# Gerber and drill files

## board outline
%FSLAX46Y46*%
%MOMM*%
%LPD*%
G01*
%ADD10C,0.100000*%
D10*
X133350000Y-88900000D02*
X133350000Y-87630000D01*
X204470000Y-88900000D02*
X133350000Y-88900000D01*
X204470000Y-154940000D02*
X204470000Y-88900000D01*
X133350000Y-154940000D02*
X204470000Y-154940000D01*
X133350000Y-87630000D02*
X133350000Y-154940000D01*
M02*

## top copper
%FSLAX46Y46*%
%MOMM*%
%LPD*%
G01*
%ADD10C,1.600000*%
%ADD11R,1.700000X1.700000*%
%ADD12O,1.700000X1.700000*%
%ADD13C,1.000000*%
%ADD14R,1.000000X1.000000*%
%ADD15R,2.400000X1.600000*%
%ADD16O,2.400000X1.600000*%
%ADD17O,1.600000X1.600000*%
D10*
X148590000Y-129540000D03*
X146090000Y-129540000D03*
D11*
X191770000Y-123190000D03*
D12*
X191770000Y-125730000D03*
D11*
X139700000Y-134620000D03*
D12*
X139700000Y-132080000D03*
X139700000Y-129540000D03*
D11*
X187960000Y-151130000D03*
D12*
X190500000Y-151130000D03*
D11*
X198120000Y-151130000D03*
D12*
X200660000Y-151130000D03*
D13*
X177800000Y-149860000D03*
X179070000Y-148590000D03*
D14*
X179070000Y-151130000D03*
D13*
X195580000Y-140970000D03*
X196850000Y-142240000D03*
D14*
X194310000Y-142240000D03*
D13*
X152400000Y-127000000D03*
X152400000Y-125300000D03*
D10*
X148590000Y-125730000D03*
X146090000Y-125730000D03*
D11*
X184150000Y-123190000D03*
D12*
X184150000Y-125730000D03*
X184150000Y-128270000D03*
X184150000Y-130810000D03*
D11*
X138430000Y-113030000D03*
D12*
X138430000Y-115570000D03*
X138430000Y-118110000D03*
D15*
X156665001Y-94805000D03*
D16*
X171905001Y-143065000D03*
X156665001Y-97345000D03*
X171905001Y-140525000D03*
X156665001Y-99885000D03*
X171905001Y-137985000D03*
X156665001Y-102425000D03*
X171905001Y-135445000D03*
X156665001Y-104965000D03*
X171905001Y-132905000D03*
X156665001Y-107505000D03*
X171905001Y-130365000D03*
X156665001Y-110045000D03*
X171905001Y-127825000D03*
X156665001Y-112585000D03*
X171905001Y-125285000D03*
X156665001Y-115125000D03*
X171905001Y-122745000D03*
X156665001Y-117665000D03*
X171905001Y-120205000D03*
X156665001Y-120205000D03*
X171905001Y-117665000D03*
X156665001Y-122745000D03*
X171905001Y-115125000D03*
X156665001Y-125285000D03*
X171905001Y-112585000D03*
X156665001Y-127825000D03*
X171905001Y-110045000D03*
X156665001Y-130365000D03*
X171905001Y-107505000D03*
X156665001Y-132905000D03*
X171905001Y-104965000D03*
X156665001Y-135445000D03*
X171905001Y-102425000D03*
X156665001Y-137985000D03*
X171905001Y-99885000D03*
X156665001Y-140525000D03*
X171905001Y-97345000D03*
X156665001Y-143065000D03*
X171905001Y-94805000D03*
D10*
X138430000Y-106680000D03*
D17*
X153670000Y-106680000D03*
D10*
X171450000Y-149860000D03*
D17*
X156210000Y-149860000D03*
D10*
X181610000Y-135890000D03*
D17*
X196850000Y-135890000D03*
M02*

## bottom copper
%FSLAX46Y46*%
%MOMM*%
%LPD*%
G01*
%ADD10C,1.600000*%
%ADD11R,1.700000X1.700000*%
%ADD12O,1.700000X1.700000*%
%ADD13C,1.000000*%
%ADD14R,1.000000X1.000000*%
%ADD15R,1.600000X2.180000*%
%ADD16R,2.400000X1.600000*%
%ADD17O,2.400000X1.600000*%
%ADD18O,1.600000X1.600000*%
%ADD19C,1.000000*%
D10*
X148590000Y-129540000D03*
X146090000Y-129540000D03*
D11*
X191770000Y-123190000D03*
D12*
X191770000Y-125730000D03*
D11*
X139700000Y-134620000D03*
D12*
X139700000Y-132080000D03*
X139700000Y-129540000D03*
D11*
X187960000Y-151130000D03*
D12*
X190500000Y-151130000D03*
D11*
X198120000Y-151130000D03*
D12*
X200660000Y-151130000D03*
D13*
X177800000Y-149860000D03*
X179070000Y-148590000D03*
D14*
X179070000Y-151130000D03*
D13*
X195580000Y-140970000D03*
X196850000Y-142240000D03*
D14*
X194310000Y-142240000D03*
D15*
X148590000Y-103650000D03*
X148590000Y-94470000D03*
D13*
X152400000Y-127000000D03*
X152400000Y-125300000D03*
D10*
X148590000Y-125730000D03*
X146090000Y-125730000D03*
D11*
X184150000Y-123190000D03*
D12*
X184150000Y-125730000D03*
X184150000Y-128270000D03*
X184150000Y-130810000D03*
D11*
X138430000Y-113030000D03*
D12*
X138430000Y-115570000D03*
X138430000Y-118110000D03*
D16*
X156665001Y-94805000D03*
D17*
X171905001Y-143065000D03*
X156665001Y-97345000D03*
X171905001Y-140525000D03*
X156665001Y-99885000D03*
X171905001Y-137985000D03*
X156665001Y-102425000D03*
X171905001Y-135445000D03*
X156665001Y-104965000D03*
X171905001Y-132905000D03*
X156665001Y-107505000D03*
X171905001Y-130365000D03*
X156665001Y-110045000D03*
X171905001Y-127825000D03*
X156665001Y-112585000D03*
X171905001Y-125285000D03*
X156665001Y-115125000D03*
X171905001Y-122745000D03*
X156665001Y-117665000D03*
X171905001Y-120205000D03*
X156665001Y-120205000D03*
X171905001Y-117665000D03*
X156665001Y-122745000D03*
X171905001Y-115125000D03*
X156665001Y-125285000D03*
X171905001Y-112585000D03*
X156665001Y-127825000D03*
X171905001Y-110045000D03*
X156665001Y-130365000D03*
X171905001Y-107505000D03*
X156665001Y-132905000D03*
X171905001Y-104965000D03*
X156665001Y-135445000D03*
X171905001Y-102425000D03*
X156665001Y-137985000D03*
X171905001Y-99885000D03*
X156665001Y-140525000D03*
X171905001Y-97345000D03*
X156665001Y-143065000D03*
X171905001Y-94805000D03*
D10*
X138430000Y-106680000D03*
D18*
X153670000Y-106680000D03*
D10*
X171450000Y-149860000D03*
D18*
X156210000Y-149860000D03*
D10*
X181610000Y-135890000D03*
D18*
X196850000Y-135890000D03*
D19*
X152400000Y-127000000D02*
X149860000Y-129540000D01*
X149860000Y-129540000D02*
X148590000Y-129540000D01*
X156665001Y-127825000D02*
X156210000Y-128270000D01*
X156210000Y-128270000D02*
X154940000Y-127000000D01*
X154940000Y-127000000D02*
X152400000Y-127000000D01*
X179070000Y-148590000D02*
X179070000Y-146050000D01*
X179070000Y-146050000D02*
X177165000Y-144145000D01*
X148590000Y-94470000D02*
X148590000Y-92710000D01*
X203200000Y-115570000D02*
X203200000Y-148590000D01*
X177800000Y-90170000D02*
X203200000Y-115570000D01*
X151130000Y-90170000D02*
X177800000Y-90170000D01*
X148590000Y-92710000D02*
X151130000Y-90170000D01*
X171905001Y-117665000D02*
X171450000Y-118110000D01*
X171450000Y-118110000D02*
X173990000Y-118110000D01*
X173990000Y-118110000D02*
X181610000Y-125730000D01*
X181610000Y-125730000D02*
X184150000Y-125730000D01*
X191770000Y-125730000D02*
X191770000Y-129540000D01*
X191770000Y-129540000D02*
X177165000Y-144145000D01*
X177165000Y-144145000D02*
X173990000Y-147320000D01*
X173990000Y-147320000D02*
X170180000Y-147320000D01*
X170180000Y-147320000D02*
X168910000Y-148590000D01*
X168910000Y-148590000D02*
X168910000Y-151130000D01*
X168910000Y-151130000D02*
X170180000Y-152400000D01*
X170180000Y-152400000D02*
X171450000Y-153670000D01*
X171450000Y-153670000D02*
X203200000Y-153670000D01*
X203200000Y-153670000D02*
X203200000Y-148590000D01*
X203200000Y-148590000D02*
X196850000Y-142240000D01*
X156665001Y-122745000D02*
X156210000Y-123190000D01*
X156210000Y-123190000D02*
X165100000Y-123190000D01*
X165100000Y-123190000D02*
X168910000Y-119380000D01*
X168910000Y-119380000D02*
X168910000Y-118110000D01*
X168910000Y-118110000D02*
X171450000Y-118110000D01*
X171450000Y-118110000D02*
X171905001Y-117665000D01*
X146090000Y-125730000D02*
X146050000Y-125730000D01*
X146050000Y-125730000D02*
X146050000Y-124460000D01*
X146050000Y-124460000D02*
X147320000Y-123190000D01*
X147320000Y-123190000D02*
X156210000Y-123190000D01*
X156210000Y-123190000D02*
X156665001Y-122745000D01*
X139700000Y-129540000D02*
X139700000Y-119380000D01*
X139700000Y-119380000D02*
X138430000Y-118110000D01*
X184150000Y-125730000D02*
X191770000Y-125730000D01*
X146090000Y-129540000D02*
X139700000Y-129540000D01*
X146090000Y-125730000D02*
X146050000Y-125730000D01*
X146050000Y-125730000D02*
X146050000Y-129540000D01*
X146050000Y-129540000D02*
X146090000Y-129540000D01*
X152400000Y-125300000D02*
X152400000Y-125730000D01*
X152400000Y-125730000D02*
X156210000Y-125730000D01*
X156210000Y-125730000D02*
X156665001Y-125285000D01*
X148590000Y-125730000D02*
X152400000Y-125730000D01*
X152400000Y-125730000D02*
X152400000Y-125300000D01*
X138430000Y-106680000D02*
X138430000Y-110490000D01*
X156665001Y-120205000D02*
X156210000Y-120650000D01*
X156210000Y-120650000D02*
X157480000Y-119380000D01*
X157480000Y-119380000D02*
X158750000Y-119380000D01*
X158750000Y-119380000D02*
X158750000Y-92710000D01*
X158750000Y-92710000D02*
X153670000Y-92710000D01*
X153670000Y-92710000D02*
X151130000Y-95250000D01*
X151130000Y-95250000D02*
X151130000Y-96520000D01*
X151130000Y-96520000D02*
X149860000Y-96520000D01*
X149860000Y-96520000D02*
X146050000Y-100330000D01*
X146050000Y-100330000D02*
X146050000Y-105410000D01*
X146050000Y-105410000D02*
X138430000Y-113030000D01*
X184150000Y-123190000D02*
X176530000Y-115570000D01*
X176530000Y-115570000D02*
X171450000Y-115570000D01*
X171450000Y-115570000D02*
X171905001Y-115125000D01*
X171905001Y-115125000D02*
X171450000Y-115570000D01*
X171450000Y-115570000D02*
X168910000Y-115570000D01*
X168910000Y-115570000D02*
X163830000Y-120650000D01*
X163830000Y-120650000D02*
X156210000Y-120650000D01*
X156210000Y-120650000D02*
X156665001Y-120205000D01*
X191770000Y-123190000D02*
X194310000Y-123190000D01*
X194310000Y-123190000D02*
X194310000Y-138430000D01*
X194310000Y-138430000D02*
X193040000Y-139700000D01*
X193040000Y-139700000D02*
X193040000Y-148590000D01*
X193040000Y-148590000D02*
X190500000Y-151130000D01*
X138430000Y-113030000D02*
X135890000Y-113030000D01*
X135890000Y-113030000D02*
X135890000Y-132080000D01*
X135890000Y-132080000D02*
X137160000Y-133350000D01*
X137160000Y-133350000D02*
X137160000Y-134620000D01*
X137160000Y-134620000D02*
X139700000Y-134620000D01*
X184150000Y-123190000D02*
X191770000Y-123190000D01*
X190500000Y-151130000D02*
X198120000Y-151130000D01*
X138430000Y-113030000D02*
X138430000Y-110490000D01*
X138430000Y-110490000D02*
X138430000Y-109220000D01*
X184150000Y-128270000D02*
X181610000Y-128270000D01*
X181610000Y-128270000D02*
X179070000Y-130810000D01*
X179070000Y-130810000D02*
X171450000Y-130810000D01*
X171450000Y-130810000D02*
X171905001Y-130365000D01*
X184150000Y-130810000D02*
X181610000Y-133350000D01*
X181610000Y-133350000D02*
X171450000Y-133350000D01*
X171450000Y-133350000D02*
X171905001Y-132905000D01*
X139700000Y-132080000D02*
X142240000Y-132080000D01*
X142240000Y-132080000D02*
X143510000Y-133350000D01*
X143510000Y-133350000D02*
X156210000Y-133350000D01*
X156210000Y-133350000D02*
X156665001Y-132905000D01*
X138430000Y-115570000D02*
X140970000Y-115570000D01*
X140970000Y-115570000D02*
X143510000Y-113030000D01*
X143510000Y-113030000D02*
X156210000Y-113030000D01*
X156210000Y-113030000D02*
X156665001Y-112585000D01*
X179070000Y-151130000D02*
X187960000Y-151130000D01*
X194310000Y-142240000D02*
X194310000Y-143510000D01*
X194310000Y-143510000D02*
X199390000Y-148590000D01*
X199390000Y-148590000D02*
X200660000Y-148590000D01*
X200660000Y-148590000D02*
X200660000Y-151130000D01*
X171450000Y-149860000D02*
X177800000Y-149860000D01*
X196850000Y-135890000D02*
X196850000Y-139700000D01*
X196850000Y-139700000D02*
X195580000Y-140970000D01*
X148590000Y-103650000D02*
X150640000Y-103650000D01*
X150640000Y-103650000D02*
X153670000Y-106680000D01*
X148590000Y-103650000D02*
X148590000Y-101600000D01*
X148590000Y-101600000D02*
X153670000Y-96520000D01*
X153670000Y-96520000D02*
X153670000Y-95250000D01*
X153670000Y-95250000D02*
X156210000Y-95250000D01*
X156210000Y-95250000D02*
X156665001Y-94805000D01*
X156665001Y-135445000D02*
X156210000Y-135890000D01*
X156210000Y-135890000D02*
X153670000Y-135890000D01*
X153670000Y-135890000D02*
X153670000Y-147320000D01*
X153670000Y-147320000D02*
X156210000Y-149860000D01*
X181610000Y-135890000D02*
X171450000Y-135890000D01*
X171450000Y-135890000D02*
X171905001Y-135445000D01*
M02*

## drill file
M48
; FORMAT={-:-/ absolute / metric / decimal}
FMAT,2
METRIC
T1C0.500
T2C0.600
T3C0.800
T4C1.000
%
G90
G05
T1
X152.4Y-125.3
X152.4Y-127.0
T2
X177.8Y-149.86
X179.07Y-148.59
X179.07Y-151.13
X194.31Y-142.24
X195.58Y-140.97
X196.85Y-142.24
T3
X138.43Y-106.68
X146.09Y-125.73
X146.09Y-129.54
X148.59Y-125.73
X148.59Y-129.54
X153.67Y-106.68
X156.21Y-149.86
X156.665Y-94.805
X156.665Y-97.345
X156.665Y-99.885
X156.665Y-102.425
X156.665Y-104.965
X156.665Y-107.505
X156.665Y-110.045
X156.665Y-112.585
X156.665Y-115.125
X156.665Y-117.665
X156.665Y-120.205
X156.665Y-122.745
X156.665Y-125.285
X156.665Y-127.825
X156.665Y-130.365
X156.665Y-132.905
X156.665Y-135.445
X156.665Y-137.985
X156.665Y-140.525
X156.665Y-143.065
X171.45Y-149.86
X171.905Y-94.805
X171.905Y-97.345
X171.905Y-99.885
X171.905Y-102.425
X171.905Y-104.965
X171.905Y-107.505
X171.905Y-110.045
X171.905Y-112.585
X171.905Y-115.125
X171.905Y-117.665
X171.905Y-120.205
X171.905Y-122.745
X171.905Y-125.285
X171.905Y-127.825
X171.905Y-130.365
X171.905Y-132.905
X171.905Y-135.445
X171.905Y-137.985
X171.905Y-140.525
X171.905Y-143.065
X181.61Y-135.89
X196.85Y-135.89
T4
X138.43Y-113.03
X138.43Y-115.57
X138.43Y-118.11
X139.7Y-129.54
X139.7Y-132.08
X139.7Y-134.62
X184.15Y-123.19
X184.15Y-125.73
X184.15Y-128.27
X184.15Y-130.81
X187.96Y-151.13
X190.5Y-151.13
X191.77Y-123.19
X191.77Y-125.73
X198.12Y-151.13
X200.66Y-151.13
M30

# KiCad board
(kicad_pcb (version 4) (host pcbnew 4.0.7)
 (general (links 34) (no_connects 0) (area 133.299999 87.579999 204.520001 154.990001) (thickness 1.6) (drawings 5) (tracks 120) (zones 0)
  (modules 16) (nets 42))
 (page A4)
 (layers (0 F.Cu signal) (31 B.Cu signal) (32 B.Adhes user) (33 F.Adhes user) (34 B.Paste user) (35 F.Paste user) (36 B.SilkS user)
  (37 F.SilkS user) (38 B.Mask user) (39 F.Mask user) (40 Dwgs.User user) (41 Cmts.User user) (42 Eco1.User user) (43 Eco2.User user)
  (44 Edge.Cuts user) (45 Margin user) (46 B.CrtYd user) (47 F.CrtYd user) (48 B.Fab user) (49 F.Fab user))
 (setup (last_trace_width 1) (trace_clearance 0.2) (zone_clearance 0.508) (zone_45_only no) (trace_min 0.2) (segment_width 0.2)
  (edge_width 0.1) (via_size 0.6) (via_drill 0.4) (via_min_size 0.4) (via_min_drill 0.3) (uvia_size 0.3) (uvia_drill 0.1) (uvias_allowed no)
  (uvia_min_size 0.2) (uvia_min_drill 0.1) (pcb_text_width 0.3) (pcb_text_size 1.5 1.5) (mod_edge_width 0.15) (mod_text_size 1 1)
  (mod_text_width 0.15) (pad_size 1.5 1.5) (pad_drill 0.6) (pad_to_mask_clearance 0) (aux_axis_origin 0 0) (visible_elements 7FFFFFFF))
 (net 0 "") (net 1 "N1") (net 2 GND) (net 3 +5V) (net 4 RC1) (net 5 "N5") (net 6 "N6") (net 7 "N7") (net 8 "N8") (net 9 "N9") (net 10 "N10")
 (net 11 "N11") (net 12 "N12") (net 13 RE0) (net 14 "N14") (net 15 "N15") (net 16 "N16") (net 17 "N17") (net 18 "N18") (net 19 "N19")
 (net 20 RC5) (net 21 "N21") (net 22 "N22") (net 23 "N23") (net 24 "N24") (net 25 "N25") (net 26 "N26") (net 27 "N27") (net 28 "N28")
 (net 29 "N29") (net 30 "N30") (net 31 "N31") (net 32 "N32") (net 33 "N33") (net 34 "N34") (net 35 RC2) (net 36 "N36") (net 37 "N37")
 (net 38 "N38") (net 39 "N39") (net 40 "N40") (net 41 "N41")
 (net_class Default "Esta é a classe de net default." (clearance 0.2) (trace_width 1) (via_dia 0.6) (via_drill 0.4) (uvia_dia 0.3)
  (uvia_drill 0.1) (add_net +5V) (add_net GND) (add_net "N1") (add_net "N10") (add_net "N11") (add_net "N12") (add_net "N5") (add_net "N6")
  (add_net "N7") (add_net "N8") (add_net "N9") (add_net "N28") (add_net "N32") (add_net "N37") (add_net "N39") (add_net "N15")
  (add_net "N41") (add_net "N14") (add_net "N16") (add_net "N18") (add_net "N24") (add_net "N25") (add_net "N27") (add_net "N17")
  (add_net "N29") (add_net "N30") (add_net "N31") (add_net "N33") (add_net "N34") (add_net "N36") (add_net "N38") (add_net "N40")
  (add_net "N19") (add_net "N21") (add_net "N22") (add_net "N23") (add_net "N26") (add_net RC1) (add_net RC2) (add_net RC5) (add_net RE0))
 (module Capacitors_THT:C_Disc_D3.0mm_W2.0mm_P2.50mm (layer F.Cu) (at 148.59 129.54 180)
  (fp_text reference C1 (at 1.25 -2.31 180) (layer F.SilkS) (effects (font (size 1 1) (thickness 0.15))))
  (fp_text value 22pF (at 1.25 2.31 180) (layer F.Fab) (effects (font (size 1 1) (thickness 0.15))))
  (pad 1 thru_hole circle (at 0 0 180) (size 1.6 1.6) (drill 0.8) (layers *.Cu *.Mask) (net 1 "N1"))
  (pad 2 thru_hole circle (at 2.5 0 180) (size 1.6 1.6) (drill 0.8) (layers *.Cu *.Mask) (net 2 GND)))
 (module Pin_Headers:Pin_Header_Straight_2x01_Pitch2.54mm (layer F.Cu) (at 191.77 123.19 270)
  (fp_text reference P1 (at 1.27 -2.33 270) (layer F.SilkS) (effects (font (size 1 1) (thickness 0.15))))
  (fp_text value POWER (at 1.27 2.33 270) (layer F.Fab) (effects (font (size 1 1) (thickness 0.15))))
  (pad 1 thru_hole rect (at 0 0 270) (size 1.7 1.7) (drill 1) (layers *.Cu *.Mask) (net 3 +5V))
  (pad 2 thru_hole oval (at 2.54 0 270) (size 1.7 1.7) (drill 1) (layers *.Cu *.Mask) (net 2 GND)))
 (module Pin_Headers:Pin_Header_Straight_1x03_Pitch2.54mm (layer F.Cu) (at 139.7 134.62 180)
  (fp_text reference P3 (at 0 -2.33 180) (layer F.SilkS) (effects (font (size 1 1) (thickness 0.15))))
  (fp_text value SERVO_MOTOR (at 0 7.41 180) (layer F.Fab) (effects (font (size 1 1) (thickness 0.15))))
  (pad 1 thru_hole rect (at 0 0 180) (size 1.7 1.7) (drill 1) (layers *.Cu *.Mask) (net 3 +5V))
  (pad 2 thru_hole oval (at 0 2.54 180) (size 1.7 1.7) (drill 1) (layers *.Cu *.Mask) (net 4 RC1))
  (pad 3 thru_hole oval (at 0 5.08 180) (size 1.7 1.7) (drill 1) (layers *.Cu *.Mask) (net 2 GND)))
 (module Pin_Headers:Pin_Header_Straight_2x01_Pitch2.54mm (layer F.Cu) (at 187.96 151.13)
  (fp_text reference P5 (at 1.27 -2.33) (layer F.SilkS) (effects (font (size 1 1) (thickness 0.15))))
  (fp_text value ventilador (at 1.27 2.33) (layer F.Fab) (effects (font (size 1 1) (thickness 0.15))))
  (pad 1 thru_hole rect (at 0 0) (size 1.7 1.7) (drill 1) (layers *.Cu *.Mask) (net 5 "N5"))
  (pad 2 thru_hole oval (at 2.54 0) (size 1.7 1.7) (drill 1) (layers *.Cu *.Mask) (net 3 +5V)))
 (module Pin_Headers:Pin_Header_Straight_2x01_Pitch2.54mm (layer F.Cu) (at 198.12 151.13)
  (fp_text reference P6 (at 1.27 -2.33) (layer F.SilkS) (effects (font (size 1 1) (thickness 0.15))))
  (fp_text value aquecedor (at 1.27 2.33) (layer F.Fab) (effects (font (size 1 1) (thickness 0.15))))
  (pad 1 thru_hole rect (at 0 0) (size 1.7 1.7) (drill 1) (layers *.Cu *.Mask) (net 3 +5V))
  (pad 2 thru_hole oval (at 2.54 0) (size 1.7 1.7) (drill 1) (layers *.Cu *.Mask) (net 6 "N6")))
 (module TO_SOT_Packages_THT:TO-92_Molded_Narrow (layer F.Cu) (at 179.07 151.13 90)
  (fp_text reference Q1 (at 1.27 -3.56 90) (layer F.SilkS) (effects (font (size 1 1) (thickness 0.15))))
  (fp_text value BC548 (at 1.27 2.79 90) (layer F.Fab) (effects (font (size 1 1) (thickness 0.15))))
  (pad 2 thru_hole circle (at 1.27 -1.27 180) (size 1 1) (drill 0.6) (layers *.Cu *.Mask) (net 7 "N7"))
  (pad 3 thru_hole circle (at 2.54 0 180) (size 1 1) (drill 0.6) (layers *.Cu *.Mask) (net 2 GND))
  (pad 1 thru_hole rect (at 0 0 180) (size 1 1) (drill 0.6) (layers *.Cu *.Mask) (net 5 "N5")))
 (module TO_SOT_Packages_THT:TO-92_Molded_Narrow (layer F.Cu) (at 194.31 142.24)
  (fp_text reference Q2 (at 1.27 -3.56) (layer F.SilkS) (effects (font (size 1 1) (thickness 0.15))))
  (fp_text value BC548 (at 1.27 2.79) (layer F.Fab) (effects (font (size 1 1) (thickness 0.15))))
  (pad 2 thru_hole circle (at 1.27 -1.27 90) (size 1 1) (drill 0.6) (layers *.Cu *.Mask) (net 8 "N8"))
  (pad 3 thru_hole circle (at 2.54 0 90) (size 1 1) (drill 0.6) (layers *.Cu *.Mask) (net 2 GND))
  (pad 1 thru_hole rect (at 0 0 90) (size 1 1) (drill 0.6) (layers *.Cu *.Mask) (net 6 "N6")))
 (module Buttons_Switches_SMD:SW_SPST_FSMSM (layer B.Cu) (at 148.59 99.06 90)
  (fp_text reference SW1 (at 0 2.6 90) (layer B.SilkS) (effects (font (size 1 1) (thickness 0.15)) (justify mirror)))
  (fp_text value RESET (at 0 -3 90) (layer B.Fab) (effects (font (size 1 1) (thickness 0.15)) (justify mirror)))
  (pad 1 smd rect (at -4.59 0 90) (size 2.18 1.6) (layers B.Cu B.Paste B.Mask) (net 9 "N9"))
  (pad 2 smd rect (at 4.59 0 90) (size 2.18 1.6) (layers B.Cu B.Paste B.Mask) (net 2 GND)))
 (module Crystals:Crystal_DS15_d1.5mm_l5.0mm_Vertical (layer F.Cu) (at 152.4 127 90)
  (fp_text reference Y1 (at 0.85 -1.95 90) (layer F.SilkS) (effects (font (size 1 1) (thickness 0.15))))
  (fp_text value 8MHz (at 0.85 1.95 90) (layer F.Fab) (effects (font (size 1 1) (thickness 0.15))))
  (pad 1 thru_hole circle (at 0 0 90) (size 1 1) (drill 0.5) (layers *.Cu *.Mask) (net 1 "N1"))
  (pad 2 thru_hole circle (at 1.7 0 90) (size 1 1) (drill 0.5) (layers *.Cu *.Mask) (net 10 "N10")))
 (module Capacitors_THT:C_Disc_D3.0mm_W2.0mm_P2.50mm (layer F.Cu) (at 148.59 125.73 180)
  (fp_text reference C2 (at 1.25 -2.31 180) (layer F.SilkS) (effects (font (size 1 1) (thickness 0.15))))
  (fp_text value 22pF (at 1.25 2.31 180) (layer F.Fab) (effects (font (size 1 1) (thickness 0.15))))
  (pad 1 thru_hole circle (at 0 0 180) (size 1.6 1.6) (drill 0.8) (layers *.Cu *.Mask) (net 10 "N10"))
  (pad 2 thru_hole circle (at 2.5 0 180) (size 1.6 1.6) (drill 0.8) (layers *.Cu *.Mask) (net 2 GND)))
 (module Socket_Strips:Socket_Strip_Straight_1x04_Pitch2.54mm (layer F.Cu) (at 184.15 123.19)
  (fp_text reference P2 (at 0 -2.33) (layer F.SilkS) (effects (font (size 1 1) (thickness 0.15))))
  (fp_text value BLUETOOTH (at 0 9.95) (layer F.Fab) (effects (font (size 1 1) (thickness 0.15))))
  (pad 1 thru_hole rect (at 0 0) (size 1.7 1.7) (drill 1) (layers *.Cu *.Mask) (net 3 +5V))
  (pad 2 thru_hole oval (at 0 2.54) (size 1.7 1.7) (drill 1) (layers *.Cu *.Mask) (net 2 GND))
  (pad 3 thru_hole oval (at 0 5.08) (size 1.7 1.7) (drill 1) (layers *.Cu *.Mask) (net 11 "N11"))
  (pad 4 thru_hole oval (at 0 7.62) (size 1.7 1.7) (drill 1) (layers *.Cu *.Mask) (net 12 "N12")))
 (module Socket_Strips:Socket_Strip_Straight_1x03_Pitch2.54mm (layer F.Cu) (at 138.43 113.03)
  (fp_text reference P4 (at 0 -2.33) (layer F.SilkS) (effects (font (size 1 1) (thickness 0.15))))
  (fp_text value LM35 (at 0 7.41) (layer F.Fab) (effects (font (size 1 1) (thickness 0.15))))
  (pad 1 thru_hole rect (at 0 0) (size 1.7 1.7) (drill 1) (layers *.Cu *.Mask) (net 3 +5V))
  (pad 2 thru_hole oval (at 0 2.54) (size 1.7 1.7) (drill 1) (layers *.Cu *.Mask) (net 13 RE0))
  (pad 3 thru_hole oval (at 0 5.08) (size 1.7 1.7) (drill 1) (layers *.Cu *.Mask) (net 2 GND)))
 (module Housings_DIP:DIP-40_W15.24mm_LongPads (layer F.Cu) (at 156.665001 94.805)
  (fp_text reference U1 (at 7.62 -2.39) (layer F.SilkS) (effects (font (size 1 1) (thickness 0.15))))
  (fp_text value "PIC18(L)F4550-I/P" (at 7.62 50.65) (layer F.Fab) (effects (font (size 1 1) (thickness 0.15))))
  (pad 1 thru_hole rect (at 0 0) (size 2.4 1.6) (drill 0.8) (layers *.Cu *.Mask) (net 9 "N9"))
  (pad 21 thru_hole oval (at 15.24 48.26) (size 2.4 1.6) (drill 0.8) (layers *.Cu *.Mask) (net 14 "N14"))
  (pad 2 thru_hole oval (at 0 2.54) (size 2.4 1.6) (drill 0.8) (layers *.Cu *.Mask) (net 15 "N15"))
  (pad 22 thru_hole oval (at 15.24 45.72) (size 2.4 1.6) (drill 0.8) (layers *.Cu *.Mask) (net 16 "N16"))
  (pad 3 thru_hole oval (at 0 5.08) (size 2.4 1.6) (drill 0.8) (layers *.Cu *.Mask) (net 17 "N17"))
  (pad 23 thru_hole oval (at 15.24 43.18) (size 2.4 1.6) (drill 0.8) (layers *.Cu *.Mask) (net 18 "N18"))
  (pad 4 thru_hole oval (at 0 7.62) (size 2.4 1.6) (drill 0.8) (layers *.Cu *.Mask) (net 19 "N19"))
  (pad 24 thru_hole oval (at 15.24 40.64) (size 2.4 1.6) (drill 0.8) (layers *.Cu *.Mask) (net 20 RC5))
  (pad 5 thru_hole oval (at 0 10.16) (size 2.4 1.6) (drill 0.8) (layers *.Cu *.Mask) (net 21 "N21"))
  (pad 25 thru_hole oval (at 15.24 38.1) (size 2.4 1.6) (drill 0.8) (layers *.Cu *.Mask) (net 12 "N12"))
  (pad 6 thru_hole oval (at 0 12.7) (size 2.4 1.6) (drill 0.8) (layers *.Cu *.Mask) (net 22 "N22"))
  (pad 26 thru_hole oval (at 15.24 35.56) (size 2.4 1.6) (drill 0.8) (layers *.Cu *.Mask) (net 11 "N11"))
  (pad 7 thru_hole oval (at 0 15.24) (size 2.4 1.6) (drill 0.8) (layers *.Cu *.Mask) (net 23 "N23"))
  (pad 27 thru_hole oval (at 15.24 33.02) (size 2.4 1.6) (drill 0.8) (layers *.Cu *.Mask) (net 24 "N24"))
  (pad 8 thru_hole oval (at 0 17.78) (size 2.4 1.6) (drill 0.8) (layers *.Cu *.Mask) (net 13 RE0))
  (pad 28 thru_hole oval (at 15.24 30.48) (size 2.4 1.6) (drill 0.8) (layers *.Cu *.Mask) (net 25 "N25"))
  (pad 9 thru_hole oval (at 0 20.32) (size 2.4 1.6) (drill 0.8) (layers *.Cu *.Mask) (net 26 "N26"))
  (pad 29 thru_hole oval (at 15.24 27.94) (size 2.4 1.6) (drill 0.8) (layers *.Cu *.Mask) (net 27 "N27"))
  (pad 10 thru_hole oval (at 0 22.86) (size 2.4 1.6) (drill 0.8) (layers *.Cu *.Mask) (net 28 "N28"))
  (pad 30 thru_hole oval (at 15.24 25.4) (size 2.4 1.6) (drill 0.8) (layers *.Cu *.Mask) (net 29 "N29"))
  (pad 11 thru_hole oval (at 0 25.4) (size 2.4 1.6) (drill 0.8) (layers *.Cu *.Mask) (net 3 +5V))
  (pad 31 thru_hole oval (at 15.24 22.86) (size 2.4 1.6) (drill 0.8) (layers *.Cu *.Mask) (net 2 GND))
  (pad 12 thru_hole oval (at 0 27.94) (size 2.4 1.6) (drill 0.8) (layers *.Cu *.Mask) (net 2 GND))
  (pad 32 thru_hole oval (at 15.24 20.32) (size 2.4 1.6) (drill 0.8) (layers *.Cu *.Mask) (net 3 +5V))
  (pad 13 thru_hole oval (at 0 30.48) (size 2.4 1.6) (drill 0.8) (layers *.Cu *.Mask) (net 10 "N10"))
  (pad 33 thru_hole oval (at 15.24 17.78) (size 2.4 1.6) (drill 0.8) (layers *.Cu *.Mask) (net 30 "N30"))
  (pad 14 thru_hole oval (at 0 33.02) (size 2.4 1.6) (drill 0.8) (layers *.Cu *.Mask) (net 1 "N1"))
  (pad 34 thru_hole oval (at 15.24 15.24) (size 2.4 1.6) (drill 0.8) (layers *.Cu *.Mask) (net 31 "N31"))
  (pad 15 thru_hole oval (at 0 35.56) (size 2.4 1.6) (drill 0.8) (layers *.Cu *.Mask) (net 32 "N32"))
  (pad 35 thru_hole oval (at 15.24 12.7) (size 2.4 1.6) (drill 0.8) (layers *.Cu *.Mask) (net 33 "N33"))
  (pad 16 thru_hole oval (at 0 38.1) (size 2.4 1.6) (drill 0.8) (layers *.Cu *.Mask) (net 4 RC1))
  (pad 36 thru_hole oval (at 15.24 10.16) (size 2.4 1.6) (drill 0.8) (layers *.Cu *.Mask) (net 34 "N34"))
  (pad 17 thru_hole oval (at 0 40.64) (size 2.4 1.6) (drill 0.8) (layers *.Cu *.Mask) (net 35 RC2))
  (pad 37 thru_hole oval (at 15.24 7.62) (size 2.4 1.6) (drill 0.8) (layers *.Cu *.Mask) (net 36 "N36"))
  (pad 18 thru_hole oval (at 0 43.18) (size 2.4 1.6) (drill 0.8) (layers *.Cu *.Mask) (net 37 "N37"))
  (pad 38 thru_hole oval (at 15.24 5.08) (size 2.4 1.6) (drill 0.8) (layers *.Cu *.Mask) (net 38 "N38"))
  (pad 19 thru_hole oval (at 0 45.72) (size 2.4 1.6) (drill 0.8) (layers *.Cu *.Mask) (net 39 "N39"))
  (pad 39 thru_hole oval (at 15.24 2.54) (size 2.4 1.6) (drill 0.8) (layers *.Cu *.Mask) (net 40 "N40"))
  (pad 20 thru_hole oval (at 0 48.26) (size 2.4 1.6) (drill 0.8) (layers *.Cu *.Mask) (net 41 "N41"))
  (pad 40 thru_hole oval (at 15.24 0) (size 2.4 1.6) (drill 0.8) (layers *.Cu *.Mask)))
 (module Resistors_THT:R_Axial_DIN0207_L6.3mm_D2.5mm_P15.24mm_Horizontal (layer F.Cu) (at 138.43 106.68)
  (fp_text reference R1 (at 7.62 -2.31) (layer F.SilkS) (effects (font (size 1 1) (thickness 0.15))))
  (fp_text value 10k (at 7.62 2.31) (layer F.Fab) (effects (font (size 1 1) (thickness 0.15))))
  (pad 1 thru_hole circle (at 0 0) (size 1.6 1.6) (drill 0.8) (layers *.Cu *.Mask) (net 3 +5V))
  (pad 2 thru_hole oval (at 15.24 0) (size 1.6 1.6) (drill 0.8) (layers *.Cu *.Mask) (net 9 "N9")))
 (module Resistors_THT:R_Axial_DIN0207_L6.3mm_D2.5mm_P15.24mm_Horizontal (layer F.Cu) (at 171.45 149.86 180)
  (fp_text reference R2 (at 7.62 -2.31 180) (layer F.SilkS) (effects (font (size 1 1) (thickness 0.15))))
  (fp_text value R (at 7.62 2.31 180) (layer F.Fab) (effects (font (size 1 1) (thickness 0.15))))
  (pad 1 thru_hole circle (at 0 0 180) (size 1.6 1.6) (drill 0.8) (layers *.Cu *.Mask) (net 7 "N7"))
  (pad 2 thru_hole oval (at 15.24 0 180) (size 1.6 1.6) (drill 0.8) (layers *.Cu *.Mask) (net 35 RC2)))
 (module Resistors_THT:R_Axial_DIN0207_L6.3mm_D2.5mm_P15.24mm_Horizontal (layer F.Cu) (at 181.61 135.89)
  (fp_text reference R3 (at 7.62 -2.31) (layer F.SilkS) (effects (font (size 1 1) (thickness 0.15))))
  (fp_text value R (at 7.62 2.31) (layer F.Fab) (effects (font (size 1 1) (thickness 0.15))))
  (pad 1 thru_hole circle (at 0 0) (size 1.6 1.6) (drill 0.8) (layers *.Cu *.Mask) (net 20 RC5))
  (pad 2 thru_hole oval (at 15.24 0) (size 1.6 1.6) (drill 0.8) (layers *.Cu *.Mask) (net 8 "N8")))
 (gr_line (start 133.35 88.9) (end 133.35 87.63) (angle 90) (layer Edge.Cuts) (width 0.1))
 (gr_line (start 204.47 88.9) (end 133.35 88.9) (angle 90) (layer Edge.Cuts) (width 0.1))
 (gr_line (start 204.47 154.94) (end 204.47 88.9) (angle 90) (layer Edge.Cuts) (width 0.1))
 (gr_line (start 133.35 154.94) (end 204.47 154.94) (angle 90) (layer Edge.Cuts) (width 0.1))
 (gr_line (start 133.35 87.63) (end 133.35 154.94) (angle 90) (layer Edge.Cuts) (width 0.1))
 (segment (start 152.4 127) (end 149.86 129.54) (width 1) (layer B.Cu) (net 1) (status 80000))
 (segment (start 149.86 129.54) (end 148.59 129.54) (width 1) (layer B.Cu) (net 1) (status 80000))
 (segment (start 156.665001 127.825) (end 156.21 128.27) (width 1) (layer B.Cu) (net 1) (status 80000))
 (segment (start 156.21 128.27) (end 154.94 127) (width 1) (layer B.Cu) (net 1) (status 80000))
 (segment (start 154.94 127) (end 152.4 127) (width 1) (layer B.Cu) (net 1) (status 80000))
 (segment (start 179.07 148.59) (end 179.07 146.05) (width 1) (layer B.Cu) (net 2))
 (segment (start 179.07 146.05) (end 177.165 144.145) (width 1) (layer B.Cu) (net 2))
 (segment (start 148.59 94.47) (end 148.59 92.71) (width 1) (layer B.Cu) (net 2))
 (segment (start 203.2 115.57) (end 203.2 148.59) (width 1) (layer B.Cu) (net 2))
 (segment (start 177.8 90.17) (end 203.2 115.57) (width 1) (layer B.Cu) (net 2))
 (segment (start 151.13 90.17) (end 177.8 90.17) (width 1) (layer B.Cu) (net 2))
 (segment (start 148.59 92.71) (end 151.13 90.17) (width 1) (layer B.Cu) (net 2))
 (segment (start 171.905001 117.665) (end 171.45 118.11) (width 1) (layer B.Cu) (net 2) (status 80000))
 (segment (start 171.45 118.11) (end 173.99 118.11) (width 1) (layer B.Cu) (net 2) (status 80000))
 (segment (start 173.99 118.11) (end 181.61 125.73) (width 1) (layer B.Cu) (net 2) (status 80000))
 (segment (start 181.61 125.73) (end 184.15 125.73) (width 1) (layer B.Cu) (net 2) (status 80000))
 (segment (start 191.77 125.73) (end 191.77 129.54) (width 1) (layer B.Cu) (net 2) (status 80000))
 (segment (start 191.77 129.54) (end 177.165 144.145) (width 1) (layer B.Cu) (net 2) (status 80000))
 (segment (start 177.165 144.145) (end 173.99 147.32) (width 1) (layer B.Cu) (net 2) (status 80000))
 (segment (start 173.99 147.32) (end 170.18 147.32) (width 1) (layer B.Cu) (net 2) (status 80000))
 (segment (start 170.18 147.32) (end 168.91 148.59) (width 1) (layer B.Cu) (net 2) (status 80000))
 (segment (start 168.91 148.59) (end 168.91 151.13) (width 1) (layer B.Cu) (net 2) (status 80000))
 (segment (start 168.91 151.13) (end 170.18 152.4) (width 1) (layer B.Cu) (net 2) (status 80000))
 (segment (start 170.18 152.4) (end 171.45 153.67) (width 1) (layer B.Cu) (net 2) (status 80000))
 (segment (start 171.45 153.67) (end 203.2 153.67) (width 1) (layer B.Cu) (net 2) (status 80000))
 (segment (start 203.2 153.67) (end 203.2 148.59) (width 1) (layer B.Cu) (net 2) (status 80000))
 (segment (start 203.2 148.59) (end 196.85 142.24) (width 1) (layer B.Cu) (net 2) (status 80000))
 (segment (start 156.665001 122.745) (end 156.21 123.19) (width 1) (layer B.Cu) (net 2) (status 80000))
 (segment (start 156.21 123.19) (end 165.1 123.19) (width 1) (layer B.Cu) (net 2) (status 80000))
 (segment (start 165.1 123.19) (end 168.91 119.38) (width 1) (layer B.Cu) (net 2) (status 80000))
 (segment (start 168.91 119.38) (end 168.91 118.11) (width 1) (layer B.Cu) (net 2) (status 80000))
 (segment (start 168.91 118.11) (end 171.45 118.11) (width 1) (layer B.Cu) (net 2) (status 80000))
 (segment (start 171.45 118.11) (end 171.905001 117.665) (width 1) (layer B.Cu) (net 2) (status 80000))
 (segment (start 146.09 125.73) (end 146.05 125.73) (width 1) (layer B.Cu) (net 2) (status 80000))
 (segment (start 146.05 125.73) (end 146.05 124.46) (width 1) (layer B.Cu) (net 2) (status 80000))
 (segment (start 146.05 124.46) (end 147.32 123.19) (width 1) (layer B.Cu) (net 2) (status 80000))
 (segment (start 147.32 123.19) (end 156.21 123.19) (width 1) (layer B.Cu) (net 2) (status 80000))
 (segment (start 156.21 123.19) (end 156.665001 122.745) (width 1) (layer B.Cu) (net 2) (status 80000))
 (segment (start 139.7 129.54) (end 139.7 119.38) (width 1) (layer B.Cu) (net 2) (status 80000))
 (segment (start 139.7 119.38) (end 138.43 118.11) (width 1) (layer B.Cu) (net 2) (status 80000))
 (segment (start 184.15 125.73) (end 191.77 125.73) (width 1) (layer B.Cu) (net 2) (status 80000))
 (segment (start 146.09 129.54) (end 139.7 129.54) (width 1) (layer B.Cu) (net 2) (status 80000))
 (segment (start 146.09 125.73) (end 146.05 125.73) (width 1) (layer B.Cu) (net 2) (status 80000))
 (segment (start 146.05 125.73) (end 146.05 129.54) (width 1) (layer B.Cu) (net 2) (status 80000))
 (segment (start 146.05 129.54) (end 146.09 129.54) (width 1) (layer B.Cu) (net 2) (status 80000))
 (segment (start 152.4 125.3) (end 152.4 125.73) (width 1) (layer B.Cu) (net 10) (status 80000))
 (segment (start 152.4 125.73) (end 156.21 125.73) (width 1) (layer B.Cu) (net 10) (status 80000))
 (segment (start 156.21 125.73) (end 156.665001 125.285) (width 1) (layer B.Cu) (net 10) (status 80000))
 (segment (start 148.59 125.73) (end 152.4 125.73) (width 1) (layer B.Cu) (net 10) (status 80000))
 (segment (start 152.4 125.73) (end 152.4 125.3) (width 1) (layer B.Cu) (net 10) (status 80000))
 (segment (start 138.43 106.68) (end 138.43 110.49) (width 1) (layer B.Cu) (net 3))
 (segment (start 156.665001 120.205) (end 156.21 120.65) (width 1) (layer B.Cu) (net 3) (status 80000))
 (segment (start 156.21 120.65) (end 157.48 119.38) (width 1) (layer B.Cu) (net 3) (status 80000))
 (segment (start 157.48 119.38) (end 158.75 119.38) (width 1) (layer B.Cu) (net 3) (status 80000))
 (segment (start 158.75 119.38) (end 158.75 92.71) (width 1) (layer B.Cu) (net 3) (status 80000))
 (segment (start 158.75 92.71) (end 153.67 92.71) (width 1) (layer B.Cu) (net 3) (status 80000))
 (segment (start 153.67 92.71) (end 151.13 95.25) (width 1) (layer B.Cu) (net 3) (status 80000))
 (segment (start 151.13 95.25) (end 151.13 96.52) (width 1) (layer B.Cu) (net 3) (status 80000))
 (segment (start 151.13 96.52) (end 149.86 96.52) (width 1) (layer B.Cu) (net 3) (status 80000))
 (segment (start 149.86 96.52) (end 146.05 100.33) (width 1) (layer B.Cu) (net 3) (status 80000))
 (segment (start 146.05 100.33) (end 146.05 105.41) (width 1) (layer B.Cu) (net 3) (status 80000))
 (segment (start 146.05 105.41) (end 138.43 113.03) (width 1) (layer B.Cu) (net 3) (status 80000))
 (segment (start 184.15 123.19) (end 176.53 115.57) (width 1) (layer B.Cu) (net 3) (status 80000))
 (segment (start 176.53 115.57) (end 171.45 115.57) (width 1) (layer B.Cu) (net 3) (status 80000))
 (segment (start 171.45 115.57) (end 171.905001 115.125) (width 1) (layer B.Cu) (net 3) (status 80000))
 (segment (start 171.905001 115.125) (end 171.45 115.57) (width 1) (layer B.Cu) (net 3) (status 80000))
 (segment (start 171.45 115.57) (end 168.91 115.57) (width 1) (layer B.Cu) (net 3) (status 80000))
 (segment (start 168.91 115.57) (end 163.83 120.65) (width 1) (layer B.Cu) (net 3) (status 80000))
 (segment (start 163.83 120.65) (end 156.21 120.65) (width 1) (layer B.Cu) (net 3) (status 80000))
 (segment (start 156.21 120.65) (end 156.665001 120.205) (width 1) (layer B.Cu) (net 3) (status 80000))
 (segment (start 191.77 123.19) (end 194.31 123.19) (width 1) (layer B.Cu) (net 3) (status 80000))
 (segment (start 194.31 123.19) (end 194.31 138.43) (width 1) (layer B.Cu) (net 3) (status 80000))
 (segment (start 194.31 138.43) (end 193.04 139.7) (width 1) (layer B.Cu) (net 3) (status 80000))
 (segment (start 193.04 139.7) (end 193.04 148.59) (width 1) (layer B.Cu) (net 3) (status 80000))
 (segment (start 193.04 148.59) (end 190.5 151.13) (width 1) (layer B.Cu) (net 3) (status 80000))
 (segment (start 138.43 113.03) (end 135.89 113.03) (width 1) (layer B.Cu) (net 3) (status 80000))
 (segment (start 135.89 113.03) (end 135.89 132.08) (width 1) (layer B.Cu) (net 3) (status 80000))
 (segment (start 135.89 132.08) (end 137.16 133.35) (width 1) (layer B.Cu) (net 3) (status 80000))
 (segment (start 137.16 133.35) (end 137.16 134.62) (width 1) (layer B.Cu) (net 3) (status 80000))
 (segment (start 137.16 134.62) (end 139.7 134.62) (width 1) (layer B.Cu) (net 3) (status 80000))
 (segment (start 184.15 123.19) (end 191.77 123.19) (width 1) (layer B.Cu) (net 3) (status 80000))
 (segment (start 190.5 151.13) (end 198.12 151.13) (width 1) (layer B.Cu) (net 3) (status 80000))
 (segment (start 138.43 113.03) (end 138.43 110.49) (width 1) (layer B.Cu) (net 3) (status 80000))
 (segment (start 138.43 110.49) (end 138.43 109.22) (width 1) (layer B.Cu) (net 3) (status 80000))
 (segment (start 184.15 128.27) (end 181.61 128.27) (width 1) (layer B.Cu) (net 11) (status 80000))
 (segment (start 181.61 128.27) (end 179.07 130.81) (width 1) (layer B.Cu) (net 11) (status 80000))
 (segment (start 179.07 130.81) (end 171.45 130.81) (width 1) (layer B.Cu) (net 11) (status 80000))
 (segment (start 171.45 130.81) (end 171.905001 130.365) (width 1) (layer B.Cu) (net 11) (status 80000))
 (segment (start 184.15 130.81) (end 181.61 133.35) (width 1) (layer B.Cu) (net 12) (status 80000))
 (segment (start 181.61 133.35) (end 171.45 133.35) (width 1) (layer B.Cu) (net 12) (status 80000))
 (segment (start 171.45 133.35) (end 171.905001 132.905) (width 1) (layer B.Cu) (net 12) (status 80000))
 (segment (start 139.7 132.08) (end 142.24 132.08) (width 1) (layer B.Cu) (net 4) (status 80000))
 (segment (start 142.24 132.08) (end 143.51 133.35) (width 1) (layer B.Cu) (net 4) (status 80000))
 (segment (start 143.51 133.35) (end 156.21 133.35) (width 1) (layer B.Cu) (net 4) (status 80000))
 (segment (start 156.21 133.35) (end 156.665001 132.905) (width 1) (layer B.Cu) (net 4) (status 80000))
 (segment (start 138.43 115.57) (end 140.97 115.57) (width 1) (layer B.Cu) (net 13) (status 80000))
 (segment (start 140.97 115.57) (end 143.51 113.03) (width 1) (layer B.Cu) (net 13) (status 80000))
 (segment (start 143.51 113.03) (end 156.21 113.03) (width 1) (layer B.Cu) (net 13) (status 80000))
 (segment (start 156.21 113.03) (end 156.665001 112.585) (width 1) (layer B.Cu) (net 13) (status 80000))
 (segment (start 179.07 151.13) (end 187.96 151.13) (width 1) (layer B.Cu) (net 5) (status 80000))
 (segment (start 194.31 142.24) (end 194.31 143.51) (width 1) (layer B.Cu) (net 6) (status 80000))
 (segment (start 194.31 143.51) (end 199.39 148.59) (width 1) (layer B.Cu) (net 6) (status 80000))
 (segment (start 199.39 148.59) (end 200.66 148.59) (width 1) (layer B.Cu) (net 6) (status 80000))
 (segment (start 200.66 148.59) (end 200.66 151.13) (width 1) (layer B.Cu) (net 6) (status 80000))
 (segment (start 171.45 149.86) (end 177.8 149.86) (width 1) (layer B.Cu) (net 7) (status 80000))
 (segment (start 196.85 135.89) (end 196.85 139.7) (width 1) (layer B.Cu) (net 8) (status 80000))
 (segment (start 196.85 139.7) (end 195.58 140.97) (width 1) (layer B.Cu) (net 8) (status 80000))
 (segment (start 148.59 103.65) (end 150.64 103.65) (width 1) (layer B.Cu) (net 9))
 (segment (start 150.64 103.65) (end 153.67 106.68) (width 1) (layer B.Cu) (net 9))
 (segment (start 148.59 103.65) (end 148.59 101.6) (width 1) (layer B.Cu) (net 9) (status 80000))
 (segment (start 148.59 101.6) (end 153.67 96.52) (width 1) (layer B.Cu) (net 9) (status 80000))
 (segment (start 153.67 96.52) (end 153.67 95.25) (width 1) (layer B.Cu) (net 9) (status 80000))
 (segment (start 153.67 95.25) (end 156.21 95.25) (width 1) (layer B.Cu) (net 9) (status 80000))
 (segment (start 156.21 95.25) (end 156.665001 94.805) (width 1) (layer B.Cu) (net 9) (status 80000))
 (segment (start 156.665001 135.445) (end 156.21 135.89) (width 1) (layer B.Cu) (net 35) (status 80000))
 (segment (start 156.21 135.89) (end 153.67 135.89) (width 1) (layer B.Cu) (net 35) (status 80000))
 (segment (start 153.67 135.89) (end 153.67 147.32) (width 1) (layer B.Cu) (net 35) (status 80000))
 (segment (start 153.67 147.32) (end 156.21 149.86) (width 1) (layer B.Cu) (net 35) (status 80000))
 (segment (start 181.61 135.89) (end 171.45 135.89) (width 1) (layer B.Cu) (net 20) (status 80000))
 (segment (start 171.45 135.89) (end 171.905001 135.445) (width 1) (layer B.Cu) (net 20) (status 80000)))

